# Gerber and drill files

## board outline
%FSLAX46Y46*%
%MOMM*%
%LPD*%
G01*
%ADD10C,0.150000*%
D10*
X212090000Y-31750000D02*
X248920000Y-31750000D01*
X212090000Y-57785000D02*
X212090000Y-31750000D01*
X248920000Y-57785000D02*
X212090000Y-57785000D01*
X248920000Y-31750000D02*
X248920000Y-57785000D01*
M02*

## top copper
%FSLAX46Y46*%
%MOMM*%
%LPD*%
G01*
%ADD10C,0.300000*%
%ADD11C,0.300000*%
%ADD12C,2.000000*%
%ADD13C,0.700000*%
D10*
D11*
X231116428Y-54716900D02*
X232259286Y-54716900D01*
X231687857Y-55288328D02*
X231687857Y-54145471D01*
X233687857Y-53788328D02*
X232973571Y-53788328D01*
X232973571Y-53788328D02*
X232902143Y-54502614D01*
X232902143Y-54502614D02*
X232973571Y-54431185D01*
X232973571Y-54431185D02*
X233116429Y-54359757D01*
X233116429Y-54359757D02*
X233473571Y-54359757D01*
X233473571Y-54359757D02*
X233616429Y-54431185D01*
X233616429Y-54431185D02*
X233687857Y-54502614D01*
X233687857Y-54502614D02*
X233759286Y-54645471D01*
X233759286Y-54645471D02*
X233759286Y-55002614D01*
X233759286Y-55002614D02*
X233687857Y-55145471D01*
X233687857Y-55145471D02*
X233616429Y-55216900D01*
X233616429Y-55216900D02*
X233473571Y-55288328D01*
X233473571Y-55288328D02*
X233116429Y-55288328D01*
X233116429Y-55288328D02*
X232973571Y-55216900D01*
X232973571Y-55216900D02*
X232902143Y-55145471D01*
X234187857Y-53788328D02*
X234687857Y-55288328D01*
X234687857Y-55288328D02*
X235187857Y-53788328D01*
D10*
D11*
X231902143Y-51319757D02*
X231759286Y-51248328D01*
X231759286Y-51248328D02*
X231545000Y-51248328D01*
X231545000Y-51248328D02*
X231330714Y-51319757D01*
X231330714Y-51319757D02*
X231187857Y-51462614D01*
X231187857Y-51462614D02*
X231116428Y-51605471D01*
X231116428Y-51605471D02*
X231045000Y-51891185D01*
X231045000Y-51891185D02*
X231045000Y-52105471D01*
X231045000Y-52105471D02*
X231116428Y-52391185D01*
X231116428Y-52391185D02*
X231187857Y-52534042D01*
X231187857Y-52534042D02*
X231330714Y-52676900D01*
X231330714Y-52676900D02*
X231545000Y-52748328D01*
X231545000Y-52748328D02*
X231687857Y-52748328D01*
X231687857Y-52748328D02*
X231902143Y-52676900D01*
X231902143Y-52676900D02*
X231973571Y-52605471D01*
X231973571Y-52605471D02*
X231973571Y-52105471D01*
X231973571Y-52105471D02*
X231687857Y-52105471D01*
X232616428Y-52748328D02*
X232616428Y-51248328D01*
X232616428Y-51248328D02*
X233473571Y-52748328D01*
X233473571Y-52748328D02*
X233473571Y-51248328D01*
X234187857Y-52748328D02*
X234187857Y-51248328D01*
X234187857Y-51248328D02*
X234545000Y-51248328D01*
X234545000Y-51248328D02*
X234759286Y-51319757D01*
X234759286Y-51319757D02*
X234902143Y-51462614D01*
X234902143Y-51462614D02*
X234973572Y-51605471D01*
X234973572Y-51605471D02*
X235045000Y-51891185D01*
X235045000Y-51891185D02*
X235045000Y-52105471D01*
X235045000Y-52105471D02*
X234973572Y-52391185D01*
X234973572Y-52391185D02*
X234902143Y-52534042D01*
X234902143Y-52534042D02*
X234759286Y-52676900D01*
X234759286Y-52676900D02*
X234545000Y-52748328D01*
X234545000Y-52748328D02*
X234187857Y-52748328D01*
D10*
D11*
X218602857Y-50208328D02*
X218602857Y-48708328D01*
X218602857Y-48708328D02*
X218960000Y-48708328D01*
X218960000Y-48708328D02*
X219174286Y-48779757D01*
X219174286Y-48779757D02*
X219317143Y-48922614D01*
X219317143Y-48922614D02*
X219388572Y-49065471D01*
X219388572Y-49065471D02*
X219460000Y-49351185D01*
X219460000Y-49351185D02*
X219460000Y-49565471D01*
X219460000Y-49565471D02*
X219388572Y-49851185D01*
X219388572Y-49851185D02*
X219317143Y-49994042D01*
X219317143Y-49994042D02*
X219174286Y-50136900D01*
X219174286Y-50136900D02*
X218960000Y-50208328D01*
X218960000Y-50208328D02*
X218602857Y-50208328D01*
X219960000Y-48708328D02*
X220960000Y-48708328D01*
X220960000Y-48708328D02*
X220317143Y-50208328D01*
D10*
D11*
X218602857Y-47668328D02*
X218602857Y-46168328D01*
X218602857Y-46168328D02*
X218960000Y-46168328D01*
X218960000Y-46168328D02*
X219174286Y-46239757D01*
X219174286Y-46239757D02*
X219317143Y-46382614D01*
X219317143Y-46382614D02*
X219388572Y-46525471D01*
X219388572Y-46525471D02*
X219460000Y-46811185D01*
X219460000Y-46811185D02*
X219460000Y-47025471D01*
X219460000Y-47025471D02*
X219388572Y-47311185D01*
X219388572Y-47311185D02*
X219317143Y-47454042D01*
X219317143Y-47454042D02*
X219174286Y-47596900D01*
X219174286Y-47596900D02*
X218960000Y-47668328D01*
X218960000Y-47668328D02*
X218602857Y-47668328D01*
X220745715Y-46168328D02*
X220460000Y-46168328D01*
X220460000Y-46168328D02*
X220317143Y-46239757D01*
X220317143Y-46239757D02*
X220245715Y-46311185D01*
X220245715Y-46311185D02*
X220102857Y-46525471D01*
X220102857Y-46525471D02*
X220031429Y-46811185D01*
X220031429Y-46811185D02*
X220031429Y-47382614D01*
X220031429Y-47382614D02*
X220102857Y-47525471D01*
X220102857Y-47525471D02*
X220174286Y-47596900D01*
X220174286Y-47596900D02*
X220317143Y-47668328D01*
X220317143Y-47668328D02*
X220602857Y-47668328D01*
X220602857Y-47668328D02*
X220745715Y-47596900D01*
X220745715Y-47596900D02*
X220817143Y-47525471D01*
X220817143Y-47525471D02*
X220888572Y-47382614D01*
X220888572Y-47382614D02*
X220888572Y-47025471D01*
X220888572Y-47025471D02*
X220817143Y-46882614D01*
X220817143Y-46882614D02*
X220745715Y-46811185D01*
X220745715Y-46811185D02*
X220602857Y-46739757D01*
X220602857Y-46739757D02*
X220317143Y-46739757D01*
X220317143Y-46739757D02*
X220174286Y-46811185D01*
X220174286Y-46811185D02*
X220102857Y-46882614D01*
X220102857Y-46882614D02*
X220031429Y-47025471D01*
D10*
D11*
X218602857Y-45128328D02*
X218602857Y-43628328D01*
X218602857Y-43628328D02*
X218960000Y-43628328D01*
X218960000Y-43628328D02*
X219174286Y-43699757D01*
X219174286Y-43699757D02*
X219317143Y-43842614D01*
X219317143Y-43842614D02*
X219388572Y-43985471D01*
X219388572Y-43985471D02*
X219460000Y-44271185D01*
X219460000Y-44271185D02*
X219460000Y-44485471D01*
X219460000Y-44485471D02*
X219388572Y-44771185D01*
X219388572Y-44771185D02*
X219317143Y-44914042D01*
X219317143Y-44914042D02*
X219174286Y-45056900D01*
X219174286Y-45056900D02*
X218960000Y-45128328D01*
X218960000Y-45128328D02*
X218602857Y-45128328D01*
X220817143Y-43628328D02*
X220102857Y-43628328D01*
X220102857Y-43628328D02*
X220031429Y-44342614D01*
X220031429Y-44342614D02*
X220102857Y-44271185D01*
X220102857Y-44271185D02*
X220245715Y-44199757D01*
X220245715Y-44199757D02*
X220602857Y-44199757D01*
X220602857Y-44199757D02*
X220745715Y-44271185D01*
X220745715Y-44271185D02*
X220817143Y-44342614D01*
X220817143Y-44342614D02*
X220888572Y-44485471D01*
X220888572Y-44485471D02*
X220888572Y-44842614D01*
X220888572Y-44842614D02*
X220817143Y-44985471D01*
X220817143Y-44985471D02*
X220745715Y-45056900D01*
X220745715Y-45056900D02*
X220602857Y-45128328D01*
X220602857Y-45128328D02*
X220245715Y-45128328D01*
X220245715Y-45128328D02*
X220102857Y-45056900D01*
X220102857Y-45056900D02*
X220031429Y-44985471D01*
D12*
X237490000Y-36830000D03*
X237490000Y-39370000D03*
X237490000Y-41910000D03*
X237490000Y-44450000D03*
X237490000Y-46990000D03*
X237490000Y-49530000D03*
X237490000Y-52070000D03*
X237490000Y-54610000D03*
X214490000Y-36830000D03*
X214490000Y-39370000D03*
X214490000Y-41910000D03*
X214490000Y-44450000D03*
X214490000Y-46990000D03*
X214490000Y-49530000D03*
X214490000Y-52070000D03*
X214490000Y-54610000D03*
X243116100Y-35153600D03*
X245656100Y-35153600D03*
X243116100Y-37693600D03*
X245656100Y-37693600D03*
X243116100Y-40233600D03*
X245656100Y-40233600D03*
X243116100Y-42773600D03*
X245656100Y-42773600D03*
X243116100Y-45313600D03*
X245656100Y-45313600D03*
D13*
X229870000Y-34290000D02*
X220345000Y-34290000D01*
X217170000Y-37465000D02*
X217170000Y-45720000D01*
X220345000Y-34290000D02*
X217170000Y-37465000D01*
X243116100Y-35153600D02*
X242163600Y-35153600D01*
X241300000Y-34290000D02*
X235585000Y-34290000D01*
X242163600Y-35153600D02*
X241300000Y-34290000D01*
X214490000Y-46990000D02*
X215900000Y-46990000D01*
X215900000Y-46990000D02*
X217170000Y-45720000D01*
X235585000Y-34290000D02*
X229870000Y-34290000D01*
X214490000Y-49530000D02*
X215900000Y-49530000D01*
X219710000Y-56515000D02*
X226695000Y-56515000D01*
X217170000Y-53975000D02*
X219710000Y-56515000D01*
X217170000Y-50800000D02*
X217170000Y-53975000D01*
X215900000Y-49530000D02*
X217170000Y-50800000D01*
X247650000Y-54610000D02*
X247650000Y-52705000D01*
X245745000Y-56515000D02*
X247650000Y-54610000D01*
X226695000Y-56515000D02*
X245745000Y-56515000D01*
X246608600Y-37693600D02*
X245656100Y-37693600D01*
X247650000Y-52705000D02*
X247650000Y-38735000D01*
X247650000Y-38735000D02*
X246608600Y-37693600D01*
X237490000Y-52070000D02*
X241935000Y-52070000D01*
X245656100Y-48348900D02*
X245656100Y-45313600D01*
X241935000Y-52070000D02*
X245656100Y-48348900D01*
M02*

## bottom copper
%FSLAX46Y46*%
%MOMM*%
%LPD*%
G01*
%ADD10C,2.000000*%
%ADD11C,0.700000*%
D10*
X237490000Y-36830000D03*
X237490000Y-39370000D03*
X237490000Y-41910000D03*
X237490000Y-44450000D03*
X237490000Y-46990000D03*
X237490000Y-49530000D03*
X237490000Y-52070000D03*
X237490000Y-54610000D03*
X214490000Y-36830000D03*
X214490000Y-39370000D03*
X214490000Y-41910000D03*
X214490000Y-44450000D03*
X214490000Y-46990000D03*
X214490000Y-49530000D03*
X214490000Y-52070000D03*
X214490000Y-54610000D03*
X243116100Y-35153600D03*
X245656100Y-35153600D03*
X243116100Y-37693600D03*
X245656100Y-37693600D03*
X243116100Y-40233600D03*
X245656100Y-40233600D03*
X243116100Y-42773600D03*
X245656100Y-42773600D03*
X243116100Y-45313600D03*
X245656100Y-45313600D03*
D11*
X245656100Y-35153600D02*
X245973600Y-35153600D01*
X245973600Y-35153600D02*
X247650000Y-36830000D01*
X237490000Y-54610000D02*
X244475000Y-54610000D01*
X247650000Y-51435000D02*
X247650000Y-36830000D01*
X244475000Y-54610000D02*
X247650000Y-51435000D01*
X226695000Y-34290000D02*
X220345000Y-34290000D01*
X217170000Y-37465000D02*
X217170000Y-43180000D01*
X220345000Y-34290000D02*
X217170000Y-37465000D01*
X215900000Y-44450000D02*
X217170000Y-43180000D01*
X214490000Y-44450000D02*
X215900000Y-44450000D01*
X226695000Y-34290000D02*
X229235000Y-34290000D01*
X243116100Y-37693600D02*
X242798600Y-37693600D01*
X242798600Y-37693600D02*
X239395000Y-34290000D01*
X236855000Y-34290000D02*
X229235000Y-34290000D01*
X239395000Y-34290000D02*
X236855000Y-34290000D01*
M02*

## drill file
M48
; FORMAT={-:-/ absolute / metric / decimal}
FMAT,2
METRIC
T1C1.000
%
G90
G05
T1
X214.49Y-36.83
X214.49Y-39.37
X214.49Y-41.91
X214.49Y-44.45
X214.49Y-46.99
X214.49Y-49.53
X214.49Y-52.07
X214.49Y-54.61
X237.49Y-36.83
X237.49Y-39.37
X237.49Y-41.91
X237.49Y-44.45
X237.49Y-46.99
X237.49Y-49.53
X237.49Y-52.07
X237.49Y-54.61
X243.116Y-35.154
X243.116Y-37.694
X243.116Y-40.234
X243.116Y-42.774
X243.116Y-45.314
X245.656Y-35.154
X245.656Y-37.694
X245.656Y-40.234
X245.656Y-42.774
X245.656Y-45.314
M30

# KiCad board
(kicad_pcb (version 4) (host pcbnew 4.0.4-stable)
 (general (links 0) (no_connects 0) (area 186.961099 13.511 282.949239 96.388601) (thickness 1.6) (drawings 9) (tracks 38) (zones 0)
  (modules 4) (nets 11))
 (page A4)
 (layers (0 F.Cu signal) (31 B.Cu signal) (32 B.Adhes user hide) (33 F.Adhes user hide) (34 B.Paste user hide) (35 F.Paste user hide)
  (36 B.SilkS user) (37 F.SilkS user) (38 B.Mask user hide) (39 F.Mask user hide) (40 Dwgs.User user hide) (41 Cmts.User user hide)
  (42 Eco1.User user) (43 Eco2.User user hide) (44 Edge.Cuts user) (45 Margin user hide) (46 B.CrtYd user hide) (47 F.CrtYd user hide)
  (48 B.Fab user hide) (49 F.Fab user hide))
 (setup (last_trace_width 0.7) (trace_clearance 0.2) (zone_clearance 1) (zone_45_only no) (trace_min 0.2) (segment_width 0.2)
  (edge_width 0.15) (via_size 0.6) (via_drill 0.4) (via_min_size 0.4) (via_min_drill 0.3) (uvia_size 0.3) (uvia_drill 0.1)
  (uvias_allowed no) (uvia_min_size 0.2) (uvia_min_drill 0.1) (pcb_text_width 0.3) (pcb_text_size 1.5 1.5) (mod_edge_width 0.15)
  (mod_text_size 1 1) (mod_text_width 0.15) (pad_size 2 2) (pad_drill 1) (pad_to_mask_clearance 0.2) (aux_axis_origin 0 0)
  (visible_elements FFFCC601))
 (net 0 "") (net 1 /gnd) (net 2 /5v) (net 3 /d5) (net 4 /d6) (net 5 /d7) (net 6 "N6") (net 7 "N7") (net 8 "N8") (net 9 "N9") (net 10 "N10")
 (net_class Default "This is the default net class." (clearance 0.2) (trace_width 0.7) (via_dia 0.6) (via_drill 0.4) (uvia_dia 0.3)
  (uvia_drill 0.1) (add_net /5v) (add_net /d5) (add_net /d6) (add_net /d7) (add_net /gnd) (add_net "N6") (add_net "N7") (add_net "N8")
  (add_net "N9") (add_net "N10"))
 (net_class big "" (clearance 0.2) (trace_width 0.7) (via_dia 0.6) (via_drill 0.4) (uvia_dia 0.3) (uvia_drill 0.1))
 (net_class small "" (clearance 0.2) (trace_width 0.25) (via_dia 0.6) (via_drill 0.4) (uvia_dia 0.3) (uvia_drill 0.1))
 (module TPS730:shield (layer F.Cu) (at 237.49 36.83)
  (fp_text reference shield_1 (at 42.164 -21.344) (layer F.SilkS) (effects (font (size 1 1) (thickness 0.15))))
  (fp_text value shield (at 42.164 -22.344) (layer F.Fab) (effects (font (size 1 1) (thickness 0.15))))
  (pad 14 thru_hole circle (at 0 0) (size 2 2) (drill 1) (layers *.Cu *.Mask))
  (pad 13 thru_hole circle (at 0 2.54) (size 2 2) (drill 1) (layers *.Cu *.Mask))
  (pad 12 thru_hole circle (at 0 5.08) (size 2 2) (drill 1) (layers *.Cu *.Mask))
  (pad 8 thru_hole circle (at 0 7.62) (size 2 2) (drill 1) (layers *.Cu *.Mask))
  (pad 7 thru_hole circle (at 0 10.16) (size 2 2) (drill 1) (layers *.Cu *.Mask))
  (pad 6 thru_hole circle (at 0 12.7) (size 2 2) (drill 1) (layers *.Cu *.Mask))
  (pad 5 thru_hole circle (at 0 15.24) (size 2 2) (drill 1) (layers *.Cu *.Mask) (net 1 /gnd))
  (pad 1 thru_hole circle (at 0 17.78) (size 2 2) (drill 1) (layers *.Cu *.Mask) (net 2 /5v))
  (pad 9 thru_hole circle (at -23 0) (size 2 2) (drill 1) (layers *.Cu *.Mask))
  (pad 10 thru_hole circle (at -23 2.54) (size 2 2) (drill 1) (layers *.Cu *.Mask))
  (pad 11 thru_hole circle (at -23 5.08) (size 2 2) (drill 1) (layers *.Cu *.Mask))
  (pad 4 thru_hole circle (at -23 7.62) (size 2 2) (drill 1) (layers *.Cu *.Mask) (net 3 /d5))
  (pad 3 thru_hole circle (at -23 10.16) (size 2 2) (drill 1) (layers *.Cu *.Mask) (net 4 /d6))
  (pad 2 thru_hole circle (at -23 12.7) (size 2 2) (drill 1) (layers *.Cu *.Mask) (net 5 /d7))
  (pad 15 thru_hole circle (at -23 15.24) (size 2 2) (drill 1) (layers *.Cu *.Mask))
  (pad 16 thru_hole circle (at -23 17.78) (size 2 2) (drill 1) (layers *.Cu *.Mask)))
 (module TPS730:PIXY (layer F.Cu) (at 250.7361 30.0736)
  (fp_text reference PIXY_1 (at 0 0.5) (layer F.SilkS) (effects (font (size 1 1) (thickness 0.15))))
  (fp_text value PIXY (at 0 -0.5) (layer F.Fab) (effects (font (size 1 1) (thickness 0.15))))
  (pad 1 thru_hole circle (at -7.62 5.08) (size 2 2) (drill 1) (layers *.Cu *.Mask) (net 4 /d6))
  (pad 2 thru_hole circle (at -5.08 5.08) (size 2 2) (drill 1) (layers *.Cu *.Mask) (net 2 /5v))
  (pad 3 thru_hole circle (at -7.62 7.62) (size 2 2) (drill 1) (layers *.Cu *.Mask) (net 3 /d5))
  (pad 4 thru_hole circle (at -5.08 7.62) (size 2 2) (drill 1) (layers *.Cu *.Mask) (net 5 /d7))
  (pad 5 thru_hole circle (at -7.62 10.16) (size 2 2) (drill 1) (layers *.Cu *.Mask) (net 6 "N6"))
  (pad 6 thru_hole circle (at -5.08 10.16) (size 2 2) (drill 1) (layers *.Cu *.Mask) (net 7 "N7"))
  (pad 7 thru_hole circle (at -7.62 12.7) (size 2 2) (drill 1) (layers *.Cu *.Mask) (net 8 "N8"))
  (pad 8 thru_hole circle (at -5.08 12.7) (size 2 2) (drill 1) (layers *.Cu *.Mask) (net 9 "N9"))
  (pad 9 thru_hole circle (at -7.62 15.24) (size 2 2) (drill 1) (layers *.Cu *.Mask) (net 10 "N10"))
  (pad 10 thru_hole circle (at -5.08 15.24) (size 2 2) (drill 1) (layers *.Cu *.Mask) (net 1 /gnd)))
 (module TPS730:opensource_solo (layer B.Cu) (at 227.33 44.45 180)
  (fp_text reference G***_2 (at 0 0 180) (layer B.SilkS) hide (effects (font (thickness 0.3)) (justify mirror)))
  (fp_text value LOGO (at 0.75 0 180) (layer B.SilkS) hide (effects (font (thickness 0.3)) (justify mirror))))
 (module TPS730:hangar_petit (layer F.Cu) (at 227.33 43.18 90)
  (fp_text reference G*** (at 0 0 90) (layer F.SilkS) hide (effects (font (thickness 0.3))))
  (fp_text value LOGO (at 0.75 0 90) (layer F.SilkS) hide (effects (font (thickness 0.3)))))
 (gr_line (start 212.09 31.75) (end 248.92 31.75) (angle 90) (layer Edge.Cuts) (width 0.15))
 (gr_line (start 212.09 57.785) (end 212.09 31.75) (angle 90) (layer Edge.Cuts) (width 0.15))
 (gr_line (start 248.92 57.785) (end 212.09 57.785) (angle 90) (layer Edge.Cuts) (width 0.15))
 (gr_line (start 248.92 31.75) (end 248.92 57.785) (angle 90) (layer Edge.Cuts) (width 0.15))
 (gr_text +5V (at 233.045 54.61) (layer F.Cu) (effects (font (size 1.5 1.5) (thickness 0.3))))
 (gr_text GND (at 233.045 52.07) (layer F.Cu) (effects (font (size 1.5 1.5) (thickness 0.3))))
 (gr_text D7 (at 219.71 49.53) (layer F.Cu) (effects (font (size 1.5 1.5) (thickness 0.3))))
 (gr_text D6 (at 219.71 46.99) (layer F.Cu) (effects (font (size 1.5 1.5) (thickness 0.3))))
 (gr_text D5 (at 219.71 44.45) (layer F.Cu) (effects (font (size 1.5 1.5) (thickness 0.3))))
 (segment (start 229.87 34.29) (end 220.345 34.29) (width 0.7) (layer F.Cu) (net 4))
 (segment (start 217.17 37.465) (end 217.17 45.72) (width 0.7) (layer F.Cu) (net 4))
 (segment (start 220.345 34.29) (end 217.17 37.465) (width 0.7) (layer F.Cu) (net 4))
 (segment (start 243.1161 35.1536) (end 242.1636 35.1536) (width 0.7) (layer F.Cu) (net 4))
 (segment (start 241.3 34.29) (end 235.585 34.29) (width 0.7) (layer F.Cu) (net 4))
 (segment (start 242.1636 35.1536) (end 241.3 34.29) (width 0.7) (layer F.Cu) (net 4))
 (segment (start 214.49 46.99) (end 215.9 46.99) (width 0.7) (layer F.Cu) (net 4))
 (segment (start 215.9 46.99) (end 217.17 45.72) (width 0.7) (layer F.Cu) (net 4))
 (segment (start 235.585 34.29) (end 229.87 34.29) (width 0.7) (layer F.Cu) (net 4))
 (segment (start 245.6561 35.1536) (end 245.9736 35.1536) (width 0.7) (layer B.Cu) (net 2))
 (segment (start 245.9736 35.1536) (end 247.65 36.83) (width 0.7) (layer B.Cu) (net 2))
 (segment (start 237.49 54.61) (end 244.475 54.61) (width 0.7) (layer B.Cu) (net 2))
 (segment (start 247.65 51.435) (end 247.65 36.83) (width 0.7) (layer B.Cu) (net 2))
 (segment (start 244.475 54.61) (end 247.65 51.435) (width 0.7) (layer B.Cu) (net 2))
 (segment (start 226.695 34.29) (end 220.345 34.29) (width 0.7) (layer B.Cu) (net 3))
 (segment (start 217.17 37.465) (end 217.17 43.18) (width 0.7) (layer B.Cu) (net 3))
 (segment (start 220.345 34.29) (end 217.17 37.465) (width 0.7) (layer B.Cu) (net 3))
 (segment (start 215.9 44.45) (end 217.17 43.18) (width 0.7) (layer B.Cu) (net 3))
 (segment (start 214.49 44.45) (end 215.9 44.45) (width 0.7) (layer B.Cu) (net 3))
 (segment (start 226.695 34.29) (end 229.235 34.29) (width 0.7) (layer B.Cu) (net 3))
 (segment (start 243.1161 37.6936) (end 242.7986 37.6936) (width 0.7) (layer B.Cu) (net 3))
 (segment (start 242.7986 37.6936) (end 239.395 34.29) (width 0.7) (layer B.Cu) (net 3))
 (segment (start 236.855 34.29) (end 229.235 34.29) (width 0.7) (layer B.Cu) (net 3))
 (segment (start 239.395 34.29) (end 236.855 34.29) (width 0.7) (layer B.Cu) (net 3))
 (segment (start 214.49 49.53) (end 215.9 49.53) (width 0.7) (layer F.Cu) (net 5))
 (segment (start 219.71 56.515) (end 226.695 56.515) (width 0.7) (layer F.Cu) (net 5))
 (segment (start 217.17 53.975) (end 219.71 56.515) (width 0.7) (layer F.Cu) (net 5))
 (segment (start 217.17 50.8) (end 217.17 53.975) (width 0.7) (layer F.Cu) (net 5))
 (segment (start 215.9 49.53) (end 217.17 50.8) (width 0.7) (layer F.Cu) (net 5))
 (segment (start 247.65 54.61) (end 247.65 52.705) (width 0.7) (layer F.Cu) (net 5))
 (segment (start 245.745 56.515) (end 247.65 54.61) (width 0.7) (layer F.Cu) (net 5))
 (segment (start 226.695 56.515) (end 245.745 56.515) (width 0.7) (layer F.Cu) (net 5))
 (segment (start 246.6086 37.6936) (end 245.6561 37.6936) (width 0.7) (layer F.Cu) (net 5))
 (segment (start 247.65 52.705) (end 247.65 38.735) (width 0.7) (layer F.Cu) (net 5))
 (segment (start 247.65 38.735) (end 246.6086 37.6936) (width 0.7) (layer F.Cu) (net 5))
 (segment (start 237.49 52.07) (end 241.935 52.07) (width 0.7) (layer F.Cu) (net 1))
 (segment (start 245.6561 48.3489) (end 245.6561 45.3136) (width 0.7) (layer F.Cu) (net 1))
 (segment (start 241.935 52.07) (end 245.6561 48.3489) (width 0.7) (layer F.Cu) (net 1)))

